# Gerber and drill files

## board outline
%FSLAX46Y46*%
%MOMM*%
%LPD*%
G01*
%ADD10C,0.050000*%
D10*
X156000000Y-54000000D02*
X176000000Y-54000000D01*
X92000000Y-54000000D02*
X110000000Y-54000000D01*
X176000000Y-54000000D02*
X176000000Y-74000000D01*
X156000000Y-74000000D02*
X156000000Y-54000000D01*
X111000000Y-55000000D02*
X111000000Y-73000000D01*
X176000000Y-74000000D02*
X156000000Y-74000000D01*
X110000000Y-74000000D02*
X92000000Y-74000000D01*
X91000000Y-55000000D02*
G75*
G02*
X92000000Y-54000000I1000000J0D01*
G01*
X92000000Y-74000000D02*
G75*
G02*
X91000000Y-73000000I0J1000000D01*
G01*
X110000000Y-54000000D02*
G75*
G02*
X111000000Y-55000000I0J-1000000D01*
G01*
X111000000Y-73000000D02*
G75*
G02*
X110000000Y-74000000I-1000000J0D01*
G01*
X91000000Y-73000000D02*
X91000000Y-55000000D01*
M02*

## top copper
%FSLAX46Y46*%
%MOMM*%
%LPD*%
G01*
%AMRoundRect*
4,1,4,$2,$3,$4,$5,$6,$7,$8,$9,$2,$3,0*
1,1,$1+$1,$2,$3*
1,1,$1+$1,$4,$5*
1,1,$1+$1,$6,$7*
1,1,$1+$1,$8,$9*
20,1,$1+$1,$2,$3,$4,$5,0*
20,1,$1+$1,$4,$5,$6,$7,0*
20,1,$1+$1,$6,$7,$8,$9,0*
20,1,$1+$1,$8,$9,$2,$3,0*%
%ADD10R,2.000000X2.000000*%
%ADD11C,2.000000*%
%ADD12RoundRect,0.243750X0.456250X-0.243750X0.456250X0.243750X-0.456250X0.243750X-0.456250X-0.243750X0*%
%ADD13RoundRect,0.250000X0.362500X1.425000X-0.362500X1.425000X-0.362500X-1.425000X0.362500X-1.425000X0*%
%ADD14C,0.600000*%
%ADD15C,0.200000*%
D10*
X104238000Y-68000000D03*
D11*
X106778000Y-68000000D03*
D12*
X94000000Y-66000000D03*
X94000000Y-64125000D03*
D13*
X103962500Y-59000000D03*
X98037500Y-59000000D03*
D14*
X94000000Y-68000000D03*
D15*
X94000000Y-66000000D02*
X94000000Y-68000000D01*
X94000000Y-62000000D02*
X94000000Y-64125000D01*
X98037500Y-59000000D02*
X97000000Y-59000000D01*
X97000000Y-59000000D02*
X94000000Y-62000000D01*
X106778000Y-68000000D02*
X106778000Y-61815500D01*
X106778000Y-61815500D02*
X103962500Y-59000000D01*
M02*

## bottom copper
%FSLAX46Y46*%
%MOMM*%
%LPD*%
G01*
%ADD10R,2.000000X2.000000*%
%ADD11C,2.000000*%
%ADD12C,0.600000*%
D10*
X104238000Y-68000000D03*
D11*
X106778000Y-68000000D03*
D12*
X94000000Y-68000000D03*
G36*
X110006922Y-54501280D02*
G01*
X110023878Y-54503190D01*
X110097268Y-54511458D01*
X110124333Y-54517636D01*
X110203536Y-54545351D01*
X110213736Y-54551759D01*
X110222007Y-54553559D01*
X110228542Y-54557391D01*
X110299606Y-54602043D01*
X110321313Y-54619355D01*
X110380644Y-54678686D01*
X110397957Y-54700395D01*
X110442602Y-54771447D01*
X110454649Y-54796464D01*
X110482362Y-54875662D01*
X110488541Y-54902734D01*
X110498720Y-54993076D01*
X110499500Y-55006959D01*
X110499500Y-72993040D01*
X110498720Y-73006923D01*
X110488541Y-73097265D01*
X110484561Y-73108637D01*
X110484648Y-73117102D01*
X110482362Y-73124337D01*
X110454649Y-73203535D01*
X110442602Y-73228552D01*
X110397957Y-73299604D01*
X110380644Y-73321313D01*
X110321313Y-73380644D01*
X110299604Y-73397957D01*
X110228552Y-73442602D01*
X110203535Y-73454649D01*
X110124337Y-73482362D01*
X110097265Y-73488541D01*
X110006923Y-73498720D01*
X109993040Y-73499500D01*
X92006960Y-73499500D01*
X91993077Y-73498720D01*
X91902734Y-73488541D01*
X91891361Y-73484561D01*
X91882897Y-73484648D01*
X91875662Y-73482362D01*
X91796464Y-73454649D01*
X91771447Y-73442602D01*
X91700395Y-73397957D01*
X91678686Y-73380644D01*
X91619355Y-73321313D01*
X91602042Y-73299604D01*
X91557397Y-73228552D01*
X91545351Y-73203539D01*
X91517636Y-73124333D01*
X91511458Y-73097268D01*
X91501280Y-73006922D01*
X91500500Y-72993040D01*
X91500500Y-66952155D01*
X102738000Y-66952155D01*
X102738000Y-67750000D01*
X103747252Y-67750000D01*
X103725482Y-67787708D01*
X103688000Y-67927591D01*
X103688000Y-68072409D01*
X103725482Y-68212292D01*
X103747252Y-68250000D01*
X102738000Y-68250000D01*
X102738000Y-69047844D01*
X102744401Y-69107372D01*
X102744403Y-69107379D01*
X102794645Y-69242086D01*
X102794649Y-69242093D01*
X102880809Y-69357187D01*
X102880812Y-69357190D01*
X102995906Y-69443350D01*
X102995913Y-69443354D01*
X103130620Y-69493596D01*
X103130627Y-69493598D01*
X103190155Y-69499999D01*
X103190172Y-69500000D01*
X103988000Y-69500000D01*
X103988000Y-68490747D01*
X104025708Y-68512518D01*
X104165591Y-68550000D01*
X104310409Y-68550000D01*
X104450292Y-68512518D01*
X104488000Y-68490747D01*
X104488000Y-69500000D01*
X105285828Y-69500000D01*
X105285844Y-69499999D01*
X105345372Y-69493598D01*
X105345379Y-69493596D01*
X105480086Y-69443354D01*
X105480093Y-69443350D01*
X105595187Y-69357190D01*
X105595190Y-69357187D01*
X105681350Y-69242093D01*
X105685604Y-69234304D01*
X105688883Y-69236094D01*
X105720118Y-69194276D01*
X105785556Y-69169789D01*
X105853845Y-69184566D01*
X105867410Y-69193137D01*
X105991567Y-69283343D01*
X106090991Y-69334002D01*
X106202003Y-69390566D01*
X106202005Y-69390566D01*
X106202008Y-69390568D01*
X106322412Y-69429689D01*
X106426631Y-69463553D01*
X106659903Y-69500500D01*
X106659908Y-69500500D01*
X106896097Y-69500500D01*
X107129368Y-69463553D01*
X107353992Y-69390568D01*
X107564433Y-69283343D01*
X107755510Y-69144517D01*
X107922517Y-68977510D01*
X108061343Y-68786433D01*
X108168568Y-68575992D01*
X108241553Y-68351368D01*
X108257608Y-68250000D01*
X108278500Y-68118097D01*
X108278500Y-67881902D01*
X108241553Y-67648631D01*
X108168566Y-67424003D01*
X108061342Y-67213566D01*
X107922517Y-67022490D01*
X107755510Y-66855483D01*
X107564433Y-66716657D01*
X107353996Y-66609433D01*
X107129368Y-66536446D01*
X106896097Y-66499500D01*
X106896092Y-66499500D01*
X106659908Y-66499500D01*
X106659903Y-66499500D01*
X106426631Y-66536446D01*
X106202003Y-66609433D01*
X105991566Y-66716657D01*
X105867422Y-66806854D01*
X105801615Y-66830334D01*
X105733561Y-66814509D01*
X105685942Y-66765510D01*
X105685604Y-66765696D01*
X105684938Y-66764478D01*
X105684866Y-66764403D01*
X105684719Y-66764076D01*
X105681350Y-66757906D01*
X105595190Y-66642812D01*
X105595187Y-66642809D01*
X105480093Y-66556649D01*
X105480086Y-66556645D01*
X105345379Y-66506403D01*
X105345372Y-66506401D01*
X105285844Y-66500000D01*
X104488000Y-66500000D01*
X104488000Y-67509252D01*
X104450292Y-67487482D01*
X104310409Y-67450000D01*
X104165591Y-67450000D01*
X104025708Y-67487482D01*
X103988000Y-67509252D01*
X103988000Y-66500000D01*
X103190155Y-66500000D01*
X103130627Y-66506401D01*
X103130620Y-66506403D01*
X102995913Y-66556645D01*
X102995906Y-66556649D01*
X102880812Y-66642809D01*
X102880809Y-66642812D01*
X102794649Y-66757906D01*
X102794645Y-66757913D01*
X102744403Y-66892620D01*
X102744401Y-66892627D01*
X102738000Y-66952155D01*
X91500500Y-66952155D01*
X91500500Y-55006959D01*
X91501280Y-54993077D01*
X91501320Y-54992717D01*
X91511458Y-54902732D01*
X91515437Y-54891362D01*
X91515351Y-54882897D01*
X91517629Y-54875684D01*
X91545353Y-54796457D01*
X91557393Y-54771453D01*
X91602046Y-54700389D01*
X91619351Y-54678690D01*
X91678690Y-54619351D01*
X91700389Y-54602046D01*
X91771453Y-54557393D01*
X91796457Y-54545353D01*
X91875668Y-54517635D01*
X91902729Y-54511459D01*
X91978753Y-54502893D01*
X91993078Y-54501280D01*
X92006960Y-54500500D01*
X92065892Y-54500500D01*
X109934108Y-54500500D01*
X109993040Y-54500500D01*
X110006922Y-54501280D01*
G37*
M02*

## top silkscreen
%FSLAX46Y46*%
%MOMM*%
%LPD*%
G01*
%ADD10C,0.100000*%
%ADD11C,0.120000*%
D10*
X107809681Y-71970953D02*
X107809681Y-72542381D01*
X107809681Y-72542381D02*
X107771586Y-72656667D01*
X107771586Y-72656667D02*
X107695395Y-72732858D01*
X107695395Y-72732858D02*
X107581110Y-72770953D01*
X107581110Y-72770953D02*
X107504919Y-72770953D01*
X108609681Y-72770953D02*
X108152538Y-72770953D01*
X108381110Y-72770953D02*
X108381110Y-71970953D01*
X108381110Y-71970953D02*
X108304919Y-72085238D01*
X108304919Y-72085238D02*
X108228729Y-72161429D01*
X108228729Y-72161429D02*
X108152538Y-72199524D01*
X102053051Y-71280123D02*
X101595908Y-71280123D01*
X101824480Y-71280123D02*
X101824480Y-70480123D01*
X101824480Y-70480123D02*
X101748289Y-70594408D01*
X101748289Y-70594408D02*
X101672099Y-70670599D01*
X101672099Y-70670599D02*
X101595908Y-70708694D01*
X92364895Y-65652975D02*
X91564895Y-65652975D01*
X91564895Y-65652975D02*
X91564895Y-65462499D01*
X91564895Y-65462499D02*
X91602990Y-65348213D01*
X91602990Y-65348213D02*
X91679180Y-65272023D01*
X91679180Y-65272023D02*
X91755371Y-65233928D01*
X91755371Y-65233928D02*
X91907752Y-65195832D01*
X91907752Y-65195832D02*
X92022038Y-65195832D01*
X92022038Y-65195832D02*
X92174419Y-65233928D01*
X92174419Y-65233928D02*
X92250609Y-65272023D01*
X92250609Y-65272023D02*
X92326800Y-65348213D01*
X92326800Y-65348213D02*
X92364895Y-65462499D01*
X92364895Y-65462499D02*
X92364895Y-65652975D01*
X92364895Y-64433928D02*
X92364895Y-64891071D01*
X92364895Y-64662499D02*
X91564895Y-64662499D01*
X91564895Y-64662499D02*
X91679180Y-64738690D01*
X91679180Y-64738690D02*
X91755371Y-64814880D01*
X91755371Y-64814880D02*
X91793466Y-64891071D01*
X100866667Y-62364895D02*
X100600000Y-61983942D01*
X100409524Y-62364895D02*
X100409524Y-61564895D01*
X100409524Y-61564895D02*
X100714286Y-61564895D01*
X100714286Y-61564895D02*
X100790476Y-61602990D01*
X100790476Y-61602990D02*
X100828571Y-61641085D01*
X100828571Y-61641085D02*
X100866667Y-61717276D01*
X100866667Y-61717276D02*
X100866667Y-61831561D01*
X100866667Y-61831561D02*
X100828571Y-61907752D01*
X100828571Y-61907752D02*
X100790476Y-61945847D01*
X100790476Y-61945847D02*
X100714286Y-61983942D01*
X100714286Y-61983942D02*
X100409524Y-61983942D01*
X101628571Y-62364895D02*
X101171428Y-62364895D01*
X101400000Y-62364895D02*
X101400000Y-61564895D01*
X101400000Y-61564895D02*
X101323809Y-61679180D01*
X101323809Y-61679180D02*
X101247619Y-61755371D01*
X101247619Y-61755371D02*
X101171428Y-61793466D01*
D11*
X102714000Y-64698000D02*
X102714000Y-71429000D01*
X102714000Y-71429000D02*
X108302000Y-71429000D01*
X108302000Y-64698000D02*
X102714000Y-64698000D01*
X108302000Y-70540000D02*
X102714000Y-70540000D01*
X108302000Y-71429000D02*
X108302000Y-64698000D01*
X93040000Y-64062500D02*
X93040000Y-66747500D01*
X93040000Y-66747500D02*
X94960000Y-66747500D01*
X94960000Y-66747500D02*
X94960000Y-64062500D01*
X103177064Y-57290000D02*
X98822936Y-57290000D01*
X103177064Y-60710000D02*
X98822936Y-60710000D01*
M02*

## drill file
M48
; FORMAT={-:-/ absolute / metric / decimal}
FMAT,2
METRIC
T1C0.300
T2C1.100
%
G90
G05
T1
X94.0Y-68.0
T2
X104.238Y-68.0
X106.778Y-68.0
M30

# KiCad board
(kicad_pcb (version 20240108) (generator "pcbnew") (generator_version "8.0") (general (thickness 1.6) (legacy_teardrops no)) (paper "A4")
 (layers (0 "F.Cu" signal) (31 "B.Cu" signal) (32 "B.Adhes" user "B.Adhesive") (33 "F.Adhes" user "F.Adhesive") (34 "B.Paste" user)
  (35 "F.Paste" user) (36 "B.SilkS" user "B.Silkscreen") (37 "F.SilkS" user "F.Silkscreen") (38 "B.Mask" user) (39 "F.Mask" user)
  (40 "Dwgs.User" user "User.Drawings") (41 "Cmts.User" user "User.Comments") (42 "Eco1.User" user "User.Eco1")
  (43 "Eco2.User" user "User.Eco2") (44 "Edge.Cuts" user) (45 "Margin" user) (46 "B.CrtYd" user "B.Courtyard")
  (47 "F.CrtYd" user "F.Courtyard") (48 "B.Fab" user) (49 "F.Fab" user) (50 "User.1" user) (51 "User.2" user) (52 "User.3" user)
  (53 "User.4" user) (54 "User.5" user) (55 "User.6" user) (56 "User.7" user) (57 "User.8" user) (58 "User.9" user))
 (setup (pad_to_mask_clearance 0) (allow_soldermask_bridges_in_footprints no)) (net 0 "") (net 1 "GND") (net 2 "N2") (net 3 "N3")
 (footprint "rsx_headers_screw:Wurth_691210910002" (layer "F.Cu") (at 105 68)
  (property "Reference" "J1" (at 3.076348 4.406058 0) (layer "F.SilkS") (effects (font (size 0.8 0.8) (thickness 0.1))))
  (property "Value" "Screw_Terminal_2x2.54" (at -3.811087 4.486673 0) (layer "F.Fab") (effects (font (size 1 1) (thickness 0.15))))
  (fp_line (start -2.286 -3.302) (end -2.286 3.429) (stroke (width 0.12) (type solid)) (layer "F.SilkS"))
  (fp_line (start -2.286 3.429) (end 3.302 3.429) (stroke (width 0.12) (type solid)) (layer "F.SilkS"))
  (fp_line (start 3.302 -3.302) (end -2.286 -3.302) (stroke (width 0.12) (type solid)) (layer "F.SilkS"))
  (fp_line (start 3.302 2.54) (end -2.286 2.54) (stroke (width 0.12) (type solid)) (layer "F.SilkS"))
  (fp_line (start 3.302 3.429) (end 3.302 -3.302) (stroke (width 0.12) (type solid)) (layer "F.SilkS"))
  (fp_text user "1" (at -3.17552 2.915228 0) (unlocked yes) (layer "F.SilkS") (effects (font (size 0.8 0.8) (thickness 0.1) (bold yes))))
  (pad "1" thru_hole rect (at -0.762 0) (size 2 2) (drill 1.1) (layers "*.Cu" "*.Mask") (remove_unused_layers no) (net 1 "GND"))
  (pad "2" thru_hole circle (at 1.778 0) (size 2 2) (drill 1.1) (layers "*.Cu" "*.Mask") (remove_unused_layers no) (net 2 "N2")))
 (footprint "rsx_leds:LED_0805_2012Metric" (layer "F.Cu") (at 94 65.0625 90)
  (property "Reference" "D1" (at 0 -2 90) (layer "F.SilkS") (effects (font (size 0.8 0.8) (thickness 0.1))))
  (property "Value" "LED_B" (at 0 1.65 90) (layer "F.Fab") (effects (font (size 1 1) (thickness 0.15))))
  (fp_line (start 1 -0.96) (end -1.685 -0.96) (stroke (width 0.12) (type solid)) (layer "F.SilkS"))
  (fp_line (start -1.685 -0.96) (end -1.685 0.96) (stroke (width 0.12) (type solid)) (layer "F.SilkS"))
  (fp_line (start -1.685 0.96) (end 1 0.96) (stroke (width 0.12) (type solid)) (layer "F.SilkS"))
  (pad "1" smd roundrect (at -0.9375 0 90) (size 0.975 1.4) (layers "F.Cu" "F.Paste" "F.Mask") (roundrect_rratio 0.25) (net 1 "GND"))
  (pad "2" smd roundrect (at 0.9375 0 90) (size 0.975 1.4) (layers "F.Cu" "F.Paste" "F.Mask") (roundrect_rratio 0.25) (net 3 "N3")))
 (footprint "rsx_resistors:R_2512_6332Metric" (layer "F.Cu") (at 101 59 180)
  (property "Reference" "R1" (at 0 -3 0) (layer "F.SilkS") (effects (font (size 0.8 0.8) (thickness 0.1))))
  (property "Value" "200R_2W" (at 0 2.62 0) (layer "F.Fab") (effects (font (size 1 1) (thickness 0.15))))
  (fp_line (start -2.177064 1.71) (end 2.177064 1.71) (stroke (width 0.12) (type solid)) (layer "F.SilkS"))
  (fp_line (start -2.177064 -1.71) (end 2.177064 -1.71) (stroke (width 0.12) (type solid)) (layer "F.SilkS"))
  (pad "1" smd roundrect (at -2.9625 0 180) (size 1.225 3.35) (layers "F.Cu" "F.Paste" "F.Mask") (roundrect_rratio 0.204082) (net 2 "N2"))
  (pad "2" smd roundrect (at 2.9625 0 180) (size 1.225 3.35) (layers "F.Cu" "F.Paste" "F.Mask") (roundrect_rratio 0.204082) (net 3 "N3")))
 (gr_line (start 156 54) (end 176 54) (stroke (width 0.05) (type default)) (layer "Edge.Cuts"))
 (gr_line (start 92 54) (end 110 54) (stroke (width 0.05) (type default)) (layer "Edge.Cuts"))
 (gr_line (start 176 54) (end 176 74) (stroke (width 0.05) (type default)) (layer "Edge.Cuts"))
 (gr_line (start 156 74) (end 156 54) (stroke (width 0.05) (type default)) (layer "Edge.Cuts"))
 (gr_line (start 111 55) (end 111 73) (stroke (width 0.05) (type default)) (layer "Edge.Cuts"))
 (gr_line (start 176 74) (end 156 74) (stroke (width 0.05) (type default)) (layer "Edge.Cuts"))
 (gr_line (start 110 74) (end 92 74) (stroke (width 0.05) (type default)) (layer "Edge.Cuts"))
 (gr_arc (start 91 55) (mid 91.292893 54.292893) (end 92 54) (stroke (width 0.05) (type default)) (layer "Edge.Cuts"))
 (gr_arc (start 92 74) (mid 91.292893 73.707107) (end 91 73) (stroke (width 0.05) (type default)) (layer "Edge.Cuts"))
 (gr_arc (start 110 54) (mid 110.707107 54.292893) (end 111 55) (stroke (width 0.05) (type default)) (layer "Edge.Cuts"))
 (gr_arc (start 111 73) (mid 110.707107 73.707107) (end 110 74) (stroke (width 0.05) (type default)) (layer "Edge.Cuts"))
 (gr_line (start 91 73) (end 91 55) (stroke (width 0.05) (type default)) (layer "Edge.Cuts"))
 (segment (start 94 66) (end 94 68) (width 0.2) (layer "F.Cu") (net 1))
 (via (at 94 68) (size 0.6) (drill 0.3) (layers "F.Cu" "B.Cu") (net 1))
 (segment (start 94 62) (end 94 64.125) (width 0.2) (layer "F.Cu") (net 3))
 (segment (start 98.0375 59) (end 97 59) (width 0.2) (layer "F.Cu") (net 3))
 (segment (start 97 59) (end 94 62) (width 0.2) (layer "F.Cu") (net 3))
 (segment (start 106.778 68) (end 106.778 61.8155) (width 0.2) (layer "F.Cu") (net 2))
 (segment (start 106.778 61.8155) (end 103.9625 59) (width 0.2) (layer "F.Cu") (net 2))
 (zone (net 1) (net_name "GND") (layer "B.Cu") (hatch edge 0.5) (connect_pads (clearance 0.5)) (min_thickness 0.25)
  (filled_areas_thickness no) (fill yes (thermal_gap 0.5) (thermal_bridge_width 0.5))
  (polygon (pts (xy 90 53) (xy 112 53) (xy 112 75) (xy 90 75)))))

